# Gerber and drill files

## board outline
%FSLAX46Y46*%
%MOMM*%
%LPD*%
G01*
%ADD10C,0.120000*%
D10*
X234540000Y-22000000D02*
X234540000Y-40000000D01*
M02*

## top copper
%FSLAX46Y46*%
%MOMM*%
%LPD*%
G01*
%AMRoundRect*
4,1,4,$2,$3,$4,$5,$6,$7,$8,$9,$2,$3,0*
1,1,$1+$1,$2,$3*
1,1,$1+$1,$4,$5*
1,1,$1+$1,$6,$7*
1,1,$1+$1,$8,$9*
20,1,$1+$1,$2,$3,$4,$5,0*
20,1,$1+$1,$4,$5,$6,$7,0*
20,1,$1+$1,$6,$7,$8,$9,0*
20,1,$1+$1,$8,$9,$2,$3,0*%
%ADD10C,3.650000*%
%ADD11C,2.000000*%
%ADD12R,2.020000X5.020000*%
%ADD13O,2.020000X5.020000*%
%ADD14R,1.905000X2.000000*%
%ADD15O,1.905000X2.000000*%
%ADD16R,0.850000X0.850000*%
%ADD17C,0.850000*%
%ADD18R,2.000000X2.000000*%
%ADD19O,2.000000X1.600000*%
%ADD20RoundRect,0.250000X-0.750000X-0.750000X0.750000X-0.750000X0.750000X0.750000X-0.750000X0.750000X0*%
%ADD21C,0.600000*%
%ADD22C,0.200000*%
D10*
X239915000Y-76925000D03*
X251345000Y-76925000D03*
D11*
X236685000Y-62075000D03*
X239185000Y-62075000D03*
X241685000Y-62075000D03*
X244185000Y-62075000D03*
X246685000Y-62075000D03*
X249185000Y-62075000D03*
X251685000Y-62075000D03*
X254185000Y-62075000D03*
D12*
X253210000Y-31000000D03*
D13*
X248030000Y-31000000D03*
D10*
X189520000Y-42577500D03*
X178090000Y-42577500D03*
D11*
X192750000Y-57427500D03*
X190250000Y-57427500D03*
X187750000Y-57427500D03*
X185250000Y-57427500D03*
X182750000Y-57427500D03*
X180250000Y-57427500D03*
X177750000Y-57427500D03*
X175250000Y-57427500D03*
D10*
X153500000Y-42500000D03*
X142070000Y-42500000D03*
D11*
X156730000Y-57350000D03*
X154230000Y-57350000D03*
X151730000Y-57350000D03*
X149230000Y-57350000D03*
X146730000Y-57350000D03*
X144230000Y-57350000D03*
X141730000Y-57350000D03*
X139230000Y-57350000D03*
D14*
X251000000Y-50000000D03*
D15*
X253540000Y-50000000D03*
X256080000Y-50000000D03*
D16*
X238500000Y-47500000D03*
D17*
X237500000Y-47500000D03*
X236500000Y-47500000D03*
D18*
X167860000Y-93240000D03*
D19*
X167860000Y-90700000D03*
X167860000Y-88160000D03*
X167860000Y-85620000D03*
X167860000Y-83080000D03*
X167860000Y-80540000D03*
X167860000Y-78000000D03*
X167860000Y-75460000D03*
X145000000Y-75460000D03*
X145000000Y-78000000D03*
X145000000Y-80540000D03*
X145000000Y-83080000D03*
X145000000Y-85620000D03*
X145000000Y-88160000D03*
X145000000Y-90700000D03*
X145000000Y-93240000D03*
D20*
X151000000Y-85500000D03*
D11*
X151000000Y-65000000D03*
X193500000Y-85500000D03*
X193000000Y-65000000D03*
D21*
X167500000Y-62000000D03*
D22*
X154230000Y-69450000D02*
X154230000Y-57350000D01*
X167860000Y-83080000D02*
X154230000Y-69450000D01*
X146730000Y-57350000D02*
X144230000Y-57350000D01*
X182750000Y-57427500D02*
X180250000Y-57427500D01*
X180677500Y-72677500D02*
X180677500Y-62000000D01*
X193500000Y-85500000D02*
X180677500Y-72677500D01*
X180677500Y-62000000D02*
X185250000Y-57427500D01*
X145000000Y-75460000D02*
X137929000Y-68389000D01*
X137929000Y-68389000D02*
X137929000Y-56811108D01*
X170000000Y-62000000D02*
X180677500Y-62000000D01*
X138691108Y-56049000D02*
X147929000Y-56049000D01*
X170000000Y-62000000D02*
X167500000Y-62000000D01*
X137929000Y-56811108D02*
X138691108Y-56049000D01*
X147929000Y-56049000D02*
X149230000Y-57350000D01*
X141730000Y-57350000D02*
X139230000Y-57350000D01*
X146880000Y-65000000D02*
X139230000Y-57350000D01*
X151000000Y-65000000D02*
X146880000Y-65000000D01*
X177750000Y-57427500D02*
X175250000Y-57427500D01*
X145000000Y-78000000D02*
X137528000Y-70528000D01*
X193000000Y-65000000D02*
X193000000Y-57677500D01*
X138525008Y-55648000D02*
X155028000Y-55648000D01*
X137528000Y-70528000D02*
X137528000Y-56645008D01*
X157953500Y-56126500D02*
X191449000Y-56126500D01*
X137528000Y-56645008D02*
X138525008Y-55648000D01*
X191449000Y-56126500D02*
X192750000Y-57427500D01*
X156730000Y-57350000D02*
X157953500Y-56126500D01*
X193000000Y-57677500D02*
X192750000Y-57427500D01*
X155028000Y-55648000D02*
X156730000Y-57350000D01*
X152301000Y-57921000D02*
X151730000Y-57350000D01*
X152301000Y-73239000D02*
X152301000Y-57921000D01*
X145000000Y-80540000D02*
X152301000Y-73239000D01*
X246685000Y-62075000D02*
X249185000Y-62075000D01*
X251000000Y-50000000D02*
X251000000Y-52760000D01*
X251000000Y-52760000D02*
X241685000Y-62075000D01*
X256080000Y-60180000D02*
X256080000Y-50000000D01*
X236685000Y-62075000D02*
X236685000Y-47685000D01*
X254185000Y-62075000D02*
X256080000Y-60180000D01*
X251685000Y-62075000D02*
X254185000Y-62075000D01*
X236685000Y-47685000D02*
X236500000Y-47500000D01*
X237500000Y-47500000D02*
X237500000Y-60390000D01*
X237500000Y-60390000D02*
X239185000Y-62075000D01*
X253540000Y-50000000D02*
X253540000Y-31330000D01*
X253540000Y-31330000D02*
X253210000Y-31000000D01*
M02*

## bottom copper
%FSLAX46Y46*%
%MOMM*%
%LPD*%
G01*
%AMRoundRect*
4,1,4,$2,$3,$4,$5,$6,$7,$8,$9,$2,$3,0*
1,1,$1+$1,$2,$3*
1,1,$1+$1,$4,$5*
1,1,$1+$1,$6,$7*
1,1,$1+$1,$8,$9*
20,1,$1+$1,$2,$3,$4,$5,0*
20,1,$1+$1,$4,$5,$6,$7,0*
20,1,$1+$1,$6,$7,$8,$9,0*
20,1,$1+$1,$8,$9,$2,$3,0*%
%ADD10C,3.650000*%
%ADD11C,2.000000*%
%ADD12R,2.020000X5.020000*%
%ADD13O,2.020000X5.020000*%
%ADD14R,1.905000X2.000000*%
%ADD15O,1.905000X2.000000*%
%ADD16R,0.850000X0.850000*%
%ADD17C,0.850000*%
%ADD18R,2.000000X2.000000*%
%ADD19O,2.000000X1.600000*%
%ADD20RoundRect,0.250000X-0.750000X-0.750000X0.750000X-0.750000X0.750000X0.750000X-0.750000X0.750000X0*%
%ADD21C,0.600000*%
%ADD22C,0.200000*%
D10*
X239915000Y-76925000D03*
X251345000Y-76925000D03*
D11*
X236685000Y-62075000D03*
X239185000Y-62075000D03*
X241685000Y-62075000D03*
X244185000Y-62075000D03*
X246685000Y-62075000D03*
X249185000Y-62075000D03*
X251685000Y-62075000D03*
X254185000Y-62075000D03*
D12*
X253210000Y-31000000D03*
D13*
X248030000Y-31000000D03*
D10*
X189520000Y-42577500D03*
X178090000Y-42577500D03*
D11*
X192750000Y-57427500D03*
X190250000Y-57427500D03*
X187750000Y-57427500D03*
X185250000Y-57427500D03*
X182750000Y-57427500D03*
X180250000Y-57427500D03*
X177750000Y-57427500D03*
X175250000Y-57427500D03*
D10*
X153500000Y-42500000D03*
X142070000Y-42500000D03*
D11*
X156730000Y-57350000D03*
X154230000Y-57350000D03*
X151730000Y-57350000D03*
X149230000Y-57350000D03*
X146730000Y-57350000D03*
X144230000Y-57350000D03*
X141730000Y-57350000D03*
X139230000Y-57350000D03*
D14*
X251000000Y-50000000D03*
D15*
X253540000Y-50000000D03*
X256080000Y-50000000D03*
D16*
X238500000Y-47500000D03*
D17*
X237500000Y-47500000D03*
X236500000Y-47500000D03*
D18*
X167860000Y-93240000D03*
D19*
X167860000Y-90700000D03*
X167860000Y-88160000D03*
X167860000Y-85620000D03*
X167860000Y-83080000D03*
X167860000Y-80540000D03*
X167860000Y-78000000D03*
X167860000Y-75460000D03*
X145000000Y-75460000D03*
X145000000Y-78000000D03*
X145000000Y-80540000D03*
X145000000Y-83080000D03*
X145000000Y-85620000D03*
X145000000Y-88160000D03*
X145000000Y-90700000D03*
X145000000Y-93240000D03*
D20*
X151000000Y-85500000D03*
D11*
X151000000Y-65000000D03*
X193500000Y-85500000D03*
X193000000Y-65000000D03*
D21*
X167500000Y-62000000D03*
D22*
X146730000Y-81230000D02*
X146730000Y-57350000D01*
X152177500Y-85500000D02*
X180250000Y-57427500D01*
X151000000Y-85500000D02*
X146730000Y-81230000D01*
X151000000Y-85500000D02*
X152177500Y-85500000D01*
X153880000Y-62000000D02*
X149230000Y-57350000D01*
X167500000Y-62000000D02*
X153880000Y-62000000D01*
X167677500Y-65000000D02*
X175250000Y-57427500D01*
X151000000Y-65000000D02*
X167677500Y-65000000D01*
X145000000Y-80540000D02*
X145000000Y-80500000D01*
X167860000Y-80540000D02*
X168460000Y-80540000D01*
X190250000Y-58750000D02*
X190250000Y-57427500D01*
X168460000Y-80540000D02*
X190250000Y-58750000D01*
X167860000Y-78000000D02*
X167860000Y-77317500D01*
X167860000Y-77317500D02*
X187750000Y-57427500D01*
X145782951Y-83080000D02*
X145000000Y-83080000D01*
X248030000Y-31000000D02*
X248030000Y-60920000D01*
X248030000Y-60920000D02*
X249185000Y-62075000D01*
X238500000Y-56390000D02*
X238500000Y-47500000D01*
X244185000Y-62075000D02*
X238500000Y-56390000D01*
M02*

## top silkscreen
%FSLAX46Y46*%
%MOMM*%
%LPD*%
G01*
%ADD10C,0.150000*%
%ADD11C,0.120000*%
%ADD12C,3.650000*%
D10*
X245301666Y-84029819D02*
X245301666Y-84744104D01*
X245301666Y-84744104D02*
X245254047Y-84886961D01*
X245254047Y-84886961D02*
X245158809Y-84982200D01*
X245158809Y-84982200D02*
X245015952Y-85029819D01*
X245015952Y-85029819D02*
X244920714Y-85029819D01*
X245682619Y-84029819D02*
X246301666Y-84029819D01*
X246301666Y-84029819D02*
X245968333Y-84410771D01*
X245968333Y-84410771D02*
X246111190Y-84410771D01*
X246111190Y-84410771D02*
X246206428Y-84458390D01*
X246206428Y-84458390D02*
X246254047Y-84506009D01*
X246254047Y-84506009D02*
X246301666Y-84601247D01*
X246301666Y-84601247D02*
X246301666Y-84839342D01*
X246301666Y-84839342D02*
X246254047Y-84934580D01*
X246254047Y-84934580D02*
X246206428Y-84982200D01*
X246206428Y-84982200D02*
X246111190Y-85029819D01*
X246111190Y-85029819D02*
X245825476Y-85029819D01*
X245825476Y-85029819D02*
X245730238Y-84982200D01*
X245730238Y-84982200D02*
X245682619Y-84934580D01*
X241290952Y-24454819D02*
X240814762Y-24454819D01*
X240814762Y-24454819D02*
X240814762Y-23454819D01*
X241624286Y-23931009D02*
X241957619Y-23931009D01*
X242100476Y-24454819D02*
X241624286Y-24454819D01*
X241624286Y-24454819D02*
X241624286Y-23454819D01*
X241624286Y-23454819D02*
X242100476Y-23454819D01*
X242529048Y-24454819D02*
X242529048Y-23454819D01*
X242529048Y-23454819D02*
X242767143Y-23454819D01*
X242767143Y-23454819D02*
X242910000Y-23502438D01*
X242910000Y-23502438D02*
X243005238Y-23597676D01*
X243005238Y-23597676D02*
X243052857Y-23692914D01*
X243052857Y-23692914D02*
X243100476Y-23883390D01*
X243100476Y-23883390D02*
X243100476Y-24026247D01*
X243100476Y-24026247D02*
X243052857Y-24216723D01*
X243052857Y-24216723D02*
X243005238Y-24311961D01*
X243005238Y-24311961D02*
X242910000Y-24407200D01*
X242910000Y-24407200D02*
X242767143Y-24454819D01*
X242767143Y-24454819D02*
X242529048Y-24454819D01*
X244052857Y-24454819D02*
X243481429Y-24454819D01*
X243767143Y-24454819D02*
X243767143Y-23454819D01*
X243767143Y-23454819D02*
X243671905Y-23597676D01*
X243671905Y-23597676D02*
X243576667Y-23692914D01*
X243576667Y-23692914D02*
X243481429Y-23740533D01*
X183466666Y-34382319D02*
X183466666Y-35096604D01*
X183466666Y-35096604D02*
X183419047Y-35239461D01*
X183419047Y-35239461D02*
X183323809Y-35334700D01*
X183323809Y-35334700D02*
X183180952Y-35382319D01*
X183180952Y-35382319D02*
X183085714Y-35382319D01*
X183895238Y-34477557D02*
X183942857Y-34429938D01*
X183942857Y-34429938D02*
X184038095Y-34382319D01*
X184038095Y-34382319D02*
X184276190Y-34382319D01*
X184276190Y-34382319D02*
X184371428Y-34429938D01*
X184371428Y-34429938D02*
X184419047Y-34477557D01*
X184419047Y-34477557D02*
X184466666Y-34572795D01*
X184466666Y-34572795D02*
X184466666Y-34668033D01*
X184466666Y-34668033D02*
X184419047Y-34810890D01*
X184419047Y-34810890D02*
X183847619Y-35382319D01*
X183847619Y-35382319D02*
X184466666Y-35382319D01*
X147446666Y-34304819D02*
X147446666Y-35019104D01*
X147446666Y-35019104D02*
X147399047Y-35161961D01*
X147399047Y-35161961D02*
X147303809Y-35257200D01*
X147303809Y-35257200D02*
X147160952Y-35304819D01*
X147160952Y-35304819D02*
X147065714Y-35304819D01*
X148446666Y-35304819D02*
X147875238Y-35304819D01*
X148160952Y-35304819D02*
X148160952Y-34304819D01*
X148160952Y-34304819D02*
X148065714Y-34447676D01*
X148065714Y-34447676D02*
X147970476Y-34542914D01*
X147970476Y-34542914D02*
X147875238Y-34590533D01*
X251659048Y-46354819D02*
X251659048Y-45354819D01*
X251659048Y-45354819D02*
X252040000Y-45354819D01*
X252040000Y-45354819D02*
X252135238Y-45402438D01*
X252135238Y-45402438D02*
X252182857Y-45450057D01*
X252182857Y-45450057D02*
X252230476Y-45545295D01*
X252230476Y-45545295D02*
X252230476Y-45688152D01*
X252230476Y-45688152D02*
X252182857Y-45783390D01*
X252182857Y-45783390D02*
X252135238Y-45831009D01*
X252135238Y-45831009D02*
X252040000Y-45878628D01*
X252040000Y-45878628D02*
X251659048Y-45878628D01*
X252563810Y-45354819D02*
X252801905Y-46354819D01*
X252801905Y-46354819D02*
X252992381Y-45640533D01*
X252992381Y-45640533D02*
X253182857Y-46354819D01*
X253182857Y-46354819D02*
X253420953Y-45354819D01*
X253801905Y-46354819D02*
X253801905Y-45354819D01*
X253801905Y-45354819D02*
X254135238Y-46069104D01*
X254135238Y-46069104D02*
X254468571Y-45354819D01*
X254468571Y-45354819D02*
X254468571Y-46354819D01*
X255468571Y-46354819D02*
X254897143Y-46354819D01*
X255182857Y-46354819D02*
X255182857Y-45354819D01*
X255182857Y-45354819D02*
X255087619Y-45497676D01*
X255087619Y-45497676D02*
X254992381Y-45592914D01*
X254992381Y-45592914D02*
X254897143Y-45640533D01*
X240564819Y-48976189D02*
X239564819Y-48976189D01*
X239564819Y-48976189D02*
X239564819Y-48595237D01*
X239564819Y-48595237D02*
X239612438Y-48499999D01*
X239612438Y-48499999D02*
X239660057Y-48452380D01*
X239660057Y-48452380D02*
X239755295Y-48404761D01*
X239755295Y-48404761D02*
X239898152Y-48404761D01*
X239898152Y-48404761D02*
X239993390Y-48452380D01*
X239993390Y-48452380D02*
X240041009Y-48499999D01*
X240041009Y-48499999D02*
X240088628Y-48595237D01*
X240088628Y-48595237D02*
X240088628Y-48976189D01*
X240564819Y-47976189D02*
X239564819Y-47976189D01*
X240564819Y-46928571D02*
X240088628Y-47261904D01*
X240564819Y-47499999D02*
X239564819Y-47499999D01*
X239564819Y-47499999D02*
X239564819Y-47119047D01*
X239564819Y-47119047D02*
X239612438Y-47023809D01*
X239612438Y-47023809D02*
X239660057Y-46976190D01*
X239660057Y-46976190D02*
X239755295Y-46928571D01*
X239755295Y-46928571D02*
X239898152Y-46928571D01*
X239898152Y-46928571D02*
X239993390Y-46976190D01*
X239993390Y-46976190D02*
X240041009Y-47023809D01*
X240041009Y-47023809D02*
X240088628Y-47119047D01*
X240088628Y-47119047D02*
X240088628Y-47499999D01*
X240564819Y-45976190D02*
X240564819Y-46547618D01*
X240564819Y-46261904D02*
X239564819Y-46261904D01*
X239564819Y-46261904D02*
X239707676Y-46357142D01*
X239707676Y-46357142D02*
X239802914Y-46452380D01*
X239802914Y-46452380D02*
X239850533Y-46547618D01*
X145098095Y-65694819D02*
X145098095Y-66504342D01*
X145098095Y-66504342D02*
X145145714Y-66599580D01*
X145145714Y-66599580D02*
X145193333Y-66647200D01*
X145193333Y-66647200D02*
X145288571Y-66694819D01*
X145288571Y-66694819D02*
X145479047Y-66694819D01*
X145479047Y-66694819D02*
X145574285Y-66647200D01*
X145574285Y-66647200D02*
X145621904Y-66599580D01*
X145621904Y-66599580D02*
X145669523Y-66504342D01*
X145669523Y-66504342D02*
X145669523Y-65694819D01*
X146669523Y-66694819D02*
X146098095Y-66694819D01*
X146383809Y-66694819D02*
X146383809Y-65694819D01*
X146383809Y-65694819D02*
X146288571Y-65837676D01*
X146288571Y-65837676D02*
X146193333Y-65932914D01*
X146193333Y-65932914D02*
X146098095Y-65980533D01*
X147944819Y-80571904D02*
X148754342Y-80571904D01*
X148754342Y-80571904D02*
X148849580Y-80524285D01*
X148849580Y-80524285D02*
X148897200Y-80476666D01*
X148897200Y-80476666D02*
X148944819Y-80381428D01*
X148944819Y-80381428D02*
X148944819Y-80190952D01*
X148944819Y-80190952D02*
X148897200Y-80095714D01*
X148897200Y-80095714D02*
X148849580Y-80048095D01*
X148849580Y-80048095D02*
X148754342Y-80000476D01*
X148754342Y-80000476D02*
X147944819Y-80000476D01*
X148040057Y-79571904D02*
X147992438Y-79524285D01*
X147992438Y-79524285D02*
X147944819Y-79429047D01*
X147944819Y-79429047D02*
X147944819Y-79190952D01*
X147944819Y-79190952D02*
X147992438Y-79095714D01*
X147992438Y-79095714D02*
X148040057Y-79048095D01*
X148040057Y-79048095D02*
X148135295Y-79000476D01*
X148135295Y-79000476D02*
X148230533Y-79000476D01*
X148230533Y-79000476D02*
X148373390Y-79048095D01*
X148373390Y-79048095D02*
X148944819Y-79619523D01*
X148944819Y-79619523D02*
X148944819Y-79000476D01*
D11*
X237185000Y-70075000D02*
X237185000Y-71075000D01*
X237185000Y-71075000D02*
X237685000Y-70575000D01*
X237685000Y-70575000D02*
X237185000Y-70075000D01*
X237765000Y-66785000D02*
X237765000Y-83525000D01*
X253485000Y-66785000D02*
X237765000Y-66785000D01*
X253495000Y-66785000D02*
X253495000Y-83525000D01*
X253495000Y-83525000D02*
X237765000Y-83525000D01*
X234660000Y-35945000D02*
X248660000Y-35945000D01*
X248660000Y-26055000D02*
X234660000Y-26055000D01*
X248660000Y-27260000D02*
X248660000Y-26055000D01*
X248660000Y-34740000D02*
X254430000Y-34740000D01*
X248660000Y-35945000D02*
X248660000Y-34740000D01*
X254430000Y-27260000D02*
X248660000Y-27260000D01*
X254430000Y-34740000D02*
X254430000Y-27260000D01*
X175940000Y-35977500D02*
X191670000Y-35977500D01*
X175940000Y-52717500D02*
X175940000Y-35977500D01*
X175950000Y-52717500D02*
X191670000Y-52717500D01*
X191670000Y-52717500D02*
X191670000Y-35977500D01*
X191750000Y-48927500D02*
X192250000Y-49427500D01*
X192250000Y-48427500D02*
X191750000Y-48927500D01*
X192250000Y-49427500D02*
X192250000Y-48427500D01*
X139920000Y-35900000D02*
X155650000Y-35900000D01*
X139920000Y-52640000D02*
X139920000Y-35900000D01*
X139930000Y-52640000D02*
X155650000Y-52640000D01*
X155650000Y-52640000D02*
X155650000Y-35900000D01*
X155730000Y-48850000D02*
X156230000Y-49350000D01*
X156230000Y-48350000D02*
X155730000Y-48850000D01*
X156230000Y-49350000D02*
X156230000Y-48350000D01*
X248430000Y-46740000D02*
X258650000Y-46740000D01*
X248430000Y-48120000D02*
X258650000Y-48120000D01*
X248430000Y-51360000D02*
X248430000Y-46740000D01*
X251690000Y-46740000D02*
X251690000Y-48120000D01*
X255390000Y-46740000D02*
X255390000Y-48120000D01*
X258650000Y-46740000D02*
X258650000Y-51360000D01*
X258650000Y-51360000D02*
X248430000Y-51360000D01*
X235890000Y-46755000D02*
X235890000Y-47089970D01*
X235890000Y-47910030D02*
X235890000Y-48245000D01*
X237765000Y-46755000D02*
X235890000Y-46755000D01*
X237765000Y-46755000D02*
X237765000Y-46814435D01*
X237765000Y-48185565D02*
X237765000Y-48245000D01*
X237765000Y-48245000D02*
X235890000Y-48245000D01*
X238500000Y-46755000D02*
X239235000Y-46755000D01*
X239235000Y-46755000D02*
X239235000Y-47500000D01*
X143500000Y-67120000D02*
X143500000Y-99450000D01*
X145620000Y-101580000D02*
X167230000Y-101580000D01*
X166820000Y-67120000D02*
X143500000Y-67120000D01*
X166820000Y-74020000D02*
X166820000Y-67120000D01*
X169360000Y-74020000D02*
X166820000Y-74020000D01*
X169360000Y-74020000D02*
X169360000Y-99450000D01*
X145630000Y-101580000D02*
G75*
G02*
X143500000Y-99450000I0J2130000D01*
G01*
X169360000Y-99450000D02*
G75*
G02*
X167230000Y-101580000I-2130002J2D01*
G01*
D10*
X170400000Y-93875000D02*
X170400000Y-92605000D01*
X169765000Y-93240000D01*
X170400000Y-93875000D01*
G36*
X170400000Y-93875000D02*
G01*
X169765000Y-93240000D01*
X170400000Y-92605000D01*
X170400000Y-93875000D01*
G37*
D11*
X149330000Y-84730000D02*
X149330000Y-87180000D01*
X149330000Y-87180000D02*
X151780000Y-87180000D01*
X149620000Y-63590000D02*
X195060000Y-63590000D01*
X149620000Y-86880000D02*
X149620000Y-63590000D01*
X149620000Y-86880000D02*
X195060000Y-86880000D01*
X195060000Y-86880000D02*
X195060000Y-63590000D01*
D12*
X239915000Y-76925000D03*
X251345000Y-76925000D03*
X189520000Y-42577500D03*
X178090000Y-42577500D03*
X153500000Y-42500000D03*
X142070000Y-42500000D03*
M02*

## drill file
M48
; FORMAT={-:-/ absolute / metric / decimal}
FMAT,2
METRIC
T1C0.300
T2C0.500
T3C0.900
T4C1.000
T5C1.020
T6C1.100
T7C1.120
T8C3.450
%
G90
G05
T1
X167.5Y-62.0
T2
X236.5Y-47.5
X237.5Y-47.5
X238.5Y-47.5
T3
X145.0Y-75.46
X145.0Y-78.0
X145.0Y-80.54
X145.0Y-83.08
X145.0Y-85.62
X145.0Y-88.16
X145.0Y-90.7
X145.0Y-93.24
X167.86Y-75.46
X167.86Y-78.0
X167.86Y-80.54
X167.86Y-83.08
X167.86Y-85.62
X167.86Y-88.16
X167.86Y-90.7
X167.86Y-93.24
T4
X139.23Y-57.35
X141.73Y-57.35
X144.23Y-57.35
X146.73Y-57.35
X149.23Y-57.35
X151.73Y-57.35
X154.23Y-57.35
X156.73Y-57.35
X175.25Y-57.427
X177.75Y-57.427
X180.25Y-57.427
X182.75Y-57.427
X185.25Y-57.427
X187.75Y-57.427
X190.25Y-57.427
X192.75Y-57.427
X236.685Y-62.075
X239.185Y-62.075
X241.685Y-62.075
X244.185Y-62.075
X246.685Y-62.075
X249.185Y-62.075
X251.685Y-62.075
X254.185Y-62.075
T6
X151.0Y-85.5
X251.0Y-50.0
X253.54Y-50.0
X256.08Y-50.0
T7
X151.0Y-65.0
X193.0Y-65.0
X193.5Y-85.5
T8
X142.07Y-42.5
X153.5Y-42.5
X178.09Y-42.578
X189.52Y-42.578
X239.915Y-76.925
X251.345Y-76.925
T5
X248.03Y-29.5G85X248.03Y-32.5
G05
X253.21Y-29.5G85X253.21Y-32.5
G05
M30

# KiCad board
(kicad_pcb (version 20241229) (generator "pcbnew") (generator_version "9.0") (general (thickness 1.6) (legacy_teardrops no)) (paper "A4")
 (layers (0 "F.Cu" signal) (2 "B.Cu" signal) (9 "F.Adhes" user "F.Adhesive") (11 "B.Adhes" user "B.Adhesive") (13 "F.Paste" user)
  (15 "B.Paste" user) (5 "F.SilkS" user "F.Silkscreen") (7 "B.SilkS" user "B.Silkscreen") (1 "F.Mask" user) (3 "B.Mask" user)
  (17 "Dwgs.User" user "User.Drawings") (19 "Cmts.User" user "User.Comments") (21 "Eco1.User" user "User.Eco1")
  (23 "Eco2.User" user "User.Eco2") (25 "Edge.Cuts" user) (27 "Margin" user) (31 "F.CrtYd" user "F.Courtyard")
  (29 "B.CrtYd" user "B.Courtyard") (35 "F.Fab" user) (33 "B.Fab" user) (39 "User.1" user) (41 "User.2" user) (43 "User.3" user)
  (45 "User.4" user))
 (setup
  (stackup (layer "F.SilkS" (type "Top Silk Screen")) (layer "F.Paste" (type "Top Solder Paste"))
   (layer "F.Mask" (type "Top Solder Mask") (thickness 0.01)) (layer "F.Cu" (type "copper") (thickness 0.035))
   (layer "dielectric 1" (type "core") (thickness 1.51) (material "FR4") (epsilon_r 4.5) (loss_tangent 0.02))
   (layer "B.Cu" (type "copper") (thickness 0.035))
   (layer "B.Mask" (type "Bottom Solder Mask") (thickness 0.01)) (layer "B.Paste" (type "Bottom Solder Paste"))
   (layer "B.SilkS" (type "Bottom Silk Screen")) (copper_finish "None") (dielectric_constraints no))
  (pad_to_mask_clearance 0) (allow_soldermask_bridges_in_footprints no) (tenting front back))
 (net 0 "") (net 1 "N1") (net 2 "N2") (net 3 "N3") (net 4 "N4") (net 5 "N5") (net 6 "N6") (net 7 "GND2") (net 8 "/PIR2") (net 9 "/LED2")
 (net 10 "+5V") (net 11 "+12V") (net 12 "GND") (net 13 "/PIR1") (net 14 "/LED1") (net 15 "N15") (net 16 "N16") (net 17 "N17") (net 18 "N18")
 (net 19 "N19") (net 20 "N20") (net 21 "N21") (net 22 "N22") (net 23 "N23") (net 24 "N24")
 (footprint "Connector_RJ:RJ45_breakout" (layer "F.Cu") (at 241.185 70.575)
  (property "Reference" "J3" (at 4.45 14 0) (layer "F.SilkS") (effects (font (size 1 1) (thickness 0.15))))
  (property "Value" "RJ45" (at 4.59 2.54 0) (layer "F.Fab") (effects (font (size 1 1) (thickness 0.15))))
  (fp_line (start -4 -0.5) (end -4 0.5) (stroke (width 0.12) (type solid)) (layer "F.SilkS"))
  (fp_line (start -4 0.5) (end -3.5 0) (stroke (width 0.12) (type solid)) (layer "F.SilkS"))
  (fp_line (start -3.5 0) (end -4 -0.5) (stroke (width 0.12) (type solid)) (layer "F.SilkS"))
  (fp_line (start -3.42 -3.79) (end -3.42 12.95) (stroke (width 0.12) (type solid)) (layer "F.SilkS"))
  (fp_line (start 12.3 -3.79) (end -3.42 -3.79) (stroke (width 0.12) (type solid)) (layer "F.SilkS"))
  (fp_line (start 12.31 -3.79) (end 12.31 12.95) (stroke (width 0.12) (type solid)) (layer "F.SilkS"))
  (fp_line (start 12.31 12.95) (end -3.42 12.95) (stroke (width 0.12) (type solid)) (layer "F.SilkS"))
  (pad "" np_thru_hole circle (at -1.27 6.35) (size 3.65 3.65) (drill 3.45) (layers "*.Cu" "*.SilkS" "*.Mask"))
  (pad "" np_thru_hole circle (at 10.16 6.35) (size 3.65 3.65) (drill 3.45) (layers "*.Cu" "*.SilkS" "*.Mask"))
  (pad "1" thru_hole circle (at -4.5 -8.5) (size 2 2) (drill 1) (layers "*.Cu" "*.Mask") (remove_unused_layers no) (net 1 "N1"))
  (pad "2" thru_hole circle (at -2 -8.5) (size 2 2) (drill 1) (layers "*.Cu" "*.Mask") (remove_unused_layers no) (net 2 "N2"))
  (pad "3" thru_hole circle (at 0.5 -8.5) (size 2 2) (drill 1) (layers "*.Cu" "*.Mask") (remove_unused_layers no) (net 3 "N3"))
  (pad "4" thru_hole circle (at 3 -8.5) (size 2 2) (drill 1) (layers "*.Cu" "*.Mask") (remove_unused_layers no) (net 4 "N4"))
  (pad "5" thru_hole circle (at 5.5 -8.5) (size 2 2) (drill 1) (layers "*.Cu" "*.Mask") (remove_unused_layers no) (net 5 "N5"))
  (pad "6" thru_hole circle (at 8 -8.5) (size 2 2) (drill 1) (layers "*.Cu" "*.Mask") (remove_unused_layers no) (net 5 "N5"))
  (pad "7" thru_hole circle (at 10.5 -8.5) (size 2 2) (drill 1) (layers "*.Cu" "*.Mask") (remove_unused_layers no) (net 1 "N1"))
  (pad "8" thru_hole circle (at 13 -8.5) (size 2 2) (drill 1) (layers "*.Cu" "*.Mask") (remove_unused_layers no) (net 1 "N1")))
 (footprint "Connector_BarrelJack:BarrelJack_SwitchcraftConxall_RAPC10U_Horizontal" (layer "F.Cu") (at 253.21 31)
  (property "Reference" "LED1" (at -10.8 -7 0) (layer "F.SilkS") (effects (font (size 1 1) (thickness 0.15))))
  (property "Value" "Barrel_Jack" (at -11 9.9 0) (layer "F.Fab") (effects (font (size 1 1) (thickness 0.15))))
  (fp_line (start -18.55 4.945) (end -4.55 4.945) (stroke (width 0.12) (type solid)) (layer "F.SilkS"))
  (fp_line (start -4.55 -4.945) (end -18.55 -4.945) (stroke (width 0.12) (type solid)) (layer "F.SilkS"))
  (fp_line (start -4.55 -3.74) (end -4.55 -4.945) (stroke (width 0.12) (type solid)) (layer "F.SilkS"))
  (fp_line (start -4.55 3.74) (end 1.22 3.74) (stroke (width 0.12) (type solid)) (layer "F.SilkS"))
  (fp_line (start -4.55 4.945) (end -4.55 3.74) (stroke (width 0.12) (type solid)) (layer "F.SilkS"))
  (fp_line (start 1.22 -3.74) (end -4.55 -3.74) (stroke (width 0.12) (type solid)) (layer "F.SilkS"))
  (fp_line (start 1.22 3.74) (end 1.22 -3.74) (stroke (width 0.12) (type solid)) (layer "F.SilkS"))
  (fp_line (start -18.67 -9) (end -18.67 9) (stroke (width 0.12) (type solid)) (layer "Edge.Cuts"))
  (pad "1" thru_hole rect (at 0 0) (size 2.02 5.02) (drill oval 1.02 4.02) (layers "*.Cu" "*.Mask") (remove_unused_layers no) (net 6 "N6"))
  (pad "2" thru_hole oval (at -5.18 0) (size 2.02 5.02) (drill oval 1.02 4.02) (layers "*.Cu" "*.Mask") (remove_unused_layers no)
   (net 5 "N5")))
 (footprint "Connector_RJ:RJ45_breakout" (layer "F.Cu") (at 188.25 48.9275 180)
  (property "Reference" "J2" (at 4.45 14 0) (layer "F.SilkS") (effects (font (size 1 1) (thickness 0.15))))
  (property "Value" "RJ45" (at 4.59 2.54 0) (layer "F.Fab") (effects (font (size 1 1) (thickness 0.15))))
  (fp_line (start 12.31 12.95) (end -3.42 12.95) (stroke (width 0.12) (type solid)) (layer "F.SilkS"))
  (fp_line (start 12.31 -3.79) (end 12.31 12.95) (stroke (width 0.12) (type solid)) (layer "F.SilkS"))
  (fp_line (start 12.3 -3.79) (end -3.42 -3.79) (stroke (width 0.12) (type solid)) (layer "F.SilkS"))
  (fp_line (start -3.42 -3.79) (end -3.42 12.95) (stroke (width 0.12) (type solid)) (layer "F.SilkS"))
  (fp_line (start -3.5 0) (end -4 -0.5) (stroke (width 0.12) (type solid)) (layer "F.SilkS"))
  (fp_line (start -4 0.5) (end -3.5 0) (stroke (width 0.12) (type solid)) (layer "F.SilkS"))
  (fp_line (start -4 -0.5) (end -4 0.5) (stroke (width 0.12) (type solid)) (layer "F.SilkS"))
  (pad "" np_thru_hole circle (at -1.27 6.35 180) (size 3.65 3.65) (drill 3.45) (layers "*.Cu" "*.SilkS" "*.Mask"))
  (pad "" np_thru_hole circle (at 10.16 6.35 180) (size 3.65 3.65) (drill 3.45) (layers "*.Cu" "*.SilkS" "*.Mask"))
  (pad "1" thru_hole circle (at -4.5 -8.5 180) (size 2 2) (drill 1) (layers "*.Cu" "*.Mask") (remove_unused_layers no) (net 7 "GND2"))
  (pad "2" thru_hole circle (at -2 -8.5 180) (size 2 2) (drill 1) (layers "*.Cu" "*.Mask") (remove_unused_layers no) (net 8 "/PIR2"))
  (pad "3" thru_hole circle (at 0.5 -8.5 180) (size 2 2) (drill 1) (layers "*.Cu" "*.Mask") (remove_unused_layers no) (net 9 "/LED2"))
  (pad "4" thru_hole circle (at 3 -8.5 180) (size 2 2) (drill 1) (layers "*.Cu" "*.Mask") (remove_unused_layers no) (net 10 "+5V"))
  (pad "5" thru_hole circle (at 5.5 -8.5 180) (size 2 2) (drill 1) (layers "*.Cu" "*.Mask") (remove_unused_layers no) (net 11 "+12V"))
  (pad "6" thru_hole circle (at 8 -8.5 180) (size 2 2) (drill 1) (layers "*.Cu" "*.Mask") (remove_unused_layers no) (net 11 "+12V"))
  (pad "7" thru_hole circle (at 10.5 -8.5 180) (size 2 2) (drill 1) (layers "*.Cu" "*.Mask") (remove_unused_layers no) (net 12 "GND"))
  (pad "8" thru_hole circle (at 13 -8.5 180) (size 2 2) (drill 1) (layers "*.Cu" "*.Mask") (remove_unused_layers no) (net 12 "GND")))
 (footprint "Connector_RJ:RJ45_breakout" (layer "F.Cu") (at 152.23 48.85 180)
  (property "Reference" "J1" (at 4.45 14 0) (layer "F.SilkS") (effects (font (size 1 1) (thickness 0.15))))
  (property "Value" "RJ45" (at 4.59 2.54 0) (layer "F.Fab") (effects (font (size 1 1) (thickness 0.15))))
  (fp_line (start 12.31 12.95) (end -3.42 12.95) (stroke (width 0.12) (type solid)) (layer "F.SilkS"))
  (fp_line (start 12.31 -3.79) (end 12.31 12.95) (stroke (width 0.12) (type solid)) (layer "F.SilkS"))
  (fp_line (start 12.3 -3.79) (end -3.42 -3.79) (stroke (width 0.12) (type solid)) (layer "F.SilkS"))
  (fp_line (start -3.42 -3.79) (end -3.42 12.95) (stroke (width 0.12) (type solid)) (layer "F.SilkS"))
  (fp_line (start -3.5 0) (end -4 -0.5) (stroke (width 0.12) (type solid)) (layer "F.SilkS"))
  (fp_line (start -4 0.5) (end -3.5 0) (stroke (width 0.12) (type solid)) (layer "F.SilkS"))
  (fp_line (start -4 -0.5) (end -4 0.5) (stroke (width 0.12) (type solid)) (layer "F.SilkS"))
  (pad "" np_thru_hole circle (at -1.27 6.35 180) (size 3.65 3.65) (drill 3.45) (layers "*.Cu" "*.SilkS" "*.Mask"))
  (pad "" np_thru_hole circle (at 10.16 6.35 180) (size 3.65 3.65) (drill 3.45) (layers "*.Cu" "*.SilkS" "*.Mask"))
  (pad "1" thru_hole circle (at -4.5 -8.5 180) (size 2 2) (drill 1) (layers "*.Cu" "*.Mask") (remove_unused_layers no) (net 7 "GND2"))
  (pad "2" thru_hole circle (at -2 -8.5 180) (size 2 2) (drill 1) (layers "*.Cu" "*.Mask") (remove_unused_layers no) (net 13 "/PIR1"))
  (pad "3" thru_hole circle (at 0.5 -8.5 180) (size 2 2) (drill 1) (layers "*.Cu" "*.Mask") (remove_unused_layers no) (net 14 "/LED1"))
  (pad "4" thru_hole circle (at 3 -8.5 180) (size 2 2) (drill 1) (layers "*.Cu" "*.Mask") (remove_unused_layers no) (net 10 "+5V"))
  (pad "5" thru_hole circle (at 5.5 -8.5 180) (size 2 2) (drill 1) (layers "*.Cu" "*.Mask") (remove_unused_layers no) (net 11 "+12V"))
  (pad "6" thru_hole circle (at 8 -8.5 180) (size 2 2) (drill 1) (layers "*.Cu" "*.Mask") (remove_unused_layers no) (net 11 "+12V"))
  (pad "7" thru_hole circle (at 10.5 -8.5 180) (size 2 2) (drill 1) (layers "*.Cu" "*.Mask") (remove_unused_layers no) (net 12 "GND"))
  (pad "8" thru_hole circle (at 13 -8.5 180) (size 2 2) (drill 1) (layers "*.Cu" "*.Mask") (remove_unused_layers no) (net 12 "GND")))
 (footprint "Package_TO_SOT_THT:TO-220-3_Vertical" (layer "F.Cu") (at 251 50)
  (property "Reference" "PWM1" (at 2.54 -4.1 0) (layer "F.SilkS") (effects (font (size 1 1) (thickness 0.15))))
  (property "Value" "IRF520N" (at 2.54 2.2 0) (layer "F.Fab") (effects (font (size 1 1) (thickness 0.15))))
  (fp_line (start -2.57 -3.26) (end 7.65 -3.26) (stroke (width 0.12) (type solid)) (layer "F.SilkS"))
  (fp_line (start -2.57 -1.88) (end 7.65 -1.88) (stroke (width 0.12) (type solid)) (layer "F.SilkS"))
  (fp_line (start -2.57 1.36) (end -2.57 -3.26) (stroke (width 0.12) (type solid)) (layer "F.SilkS"))
  (fp_line (start 0.69 -3.26) (end 0.69 -1.88) (stroke (width 0.12) (type solid)) (layer "F.SilkS"))
  (fp_line (start 4.39 -3.26) (end 4.39 -1.88) (stroke (width 0.12) (type solid)) (layer "F.SilkS"))
  (fp_line (start 7.65 -3.26) (end 7.65 1.36) (stroke (width 0.12) (type solid)) (layer "F.SilkS"))
  (fp_line (start 7.65 1.36) (end -2.57 1.36) (stroke (width 0.12) (type solid)) (layer "F.SilkS"))
  (pad "1" thru_hole rect (at 0 0) (size 1.905 2) (drill 1.1) (layers "*.Cu" "*.Mask") (remove_unused_layers no) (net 3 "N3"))
  (pad "2" thru_hole oval (at 2.54 0) (size 1.905 2) (drill 1.1) (layers "*.Cu" "*.Mask") (remove_unused_layers no) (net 6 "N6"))
  (pad "3" thru_hole oval (at 5.08 0) (size 1.905 2) (drill 1.1) (layers "*.Cu" "*.Mask") (remove_unused_layers no) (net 1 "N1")))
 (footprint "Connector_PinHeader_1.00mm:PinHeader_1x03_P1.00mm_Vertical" (layer "F.Cu") (at 238.5 47.5 -90)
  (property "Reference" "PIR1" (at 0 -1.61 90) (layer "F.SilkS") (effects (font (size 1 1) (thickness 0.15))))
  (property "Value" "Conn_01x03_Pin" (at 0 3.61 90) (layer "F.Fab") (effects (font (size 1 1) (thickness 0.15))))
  (fp_line (start -0.745 2.61) (end -0.41003 2.61) (stroke (width 0.12) (type solid)) (layer "F.SilkS"))
  (fp_line (start 0.41003 2.61) (end 0.745 2.61) (stroke (width 0.12) (type solid)) (layer "F.SilkS"))
  (fp_line (start -0.745 0.735) (end -0.745 2.61) (stroke (width 0.12) (type solid)) (layer "F.SilkS"))
  (fp_line (start -0.745 0.735) (end -0.685565 0.735) (stroke (width 0.12) (type solid)) (layer "F.SilkS"))
  (fp_line (start 0.685565 0.735) (end 0.745 0.735) (stroke (width 0.12) (type solid)) (layer "F.SilkS"))
  (fp_line (start 0.745 0.735) (end 0.745 2.61) (stroke (width 0.12) (type solid)) (layer "F.SilkS"))
  (fp_line (start -0.745 0) (end -0.745 -0.735) (stroke (width 0.12) (type solid)) (layer "F.SilkS"))
  (fp_line (start -0.745 -0.735) (end 0 -0.735) (stroke (width 0.12) (type solid)) (layer "F.SilkS"))
  (pad "1" thru_hole rect (at 0 0 270) (size 0.85 0.85) (drill 0.5) (layers "*.Cu" "*.Mask") (remove_unused_layers no) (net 4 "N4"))
  (pad "2" thru_hole circle (at 0 1 270) (size 0.85 0.85) (drill 0.5) (layers "*.Cu" "*.Mask") (remove_unused_layers no) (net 2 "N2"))
  (pad "3" thru_hole circle (at 0 2 270) (size 0.85 0.85) (drill 0.5) (layers "*.Cu" "*.Mask") (remove_unused_layers no) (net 1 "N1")))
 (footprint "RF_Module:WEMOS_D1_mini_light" (layer "F.Cu") (at 167.86 93.24 180)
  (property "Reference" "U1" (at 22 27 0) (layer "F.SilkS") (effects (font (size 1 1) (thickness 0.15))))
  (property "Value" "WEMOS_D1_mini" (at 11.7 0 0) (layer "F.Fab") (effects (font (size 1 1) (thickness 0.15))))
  (fp_line (start 24.36 26.12) (end 24.36 -6.21) (stroke (width 0.12) (type solid)) (layer "F.SilkS"))
  (fp_line (start 22.24 -8.34) (end 0.63 -8.34) (stroke (width 0.12) (type solid)) (layer "F.SilkS"))
  (fp_line (start 1.04 26.12) (end 24.36 26.12) (stroke (width 0.12) (type solid)) (layer "F.SilkS"))
  (fp_line (start 1.04 19.22) (end 1.04 26.12) (stroke (width 0.12) (type solid)) (layer "F.SilkS"))
  (fp_line (start -1.5 19.22) (end 1.04 19.22) (stroke (width 0.12) (type solid)) (layer "F.SilkS"))
  (fp_line (start -1.5 19.22) (end -1.5 -6.21) (stroke (width 0.12) (type solid)) (layer "F.SilkS"))
  (fp_arc (start 22.23 -8.34) (mid 23.736137 -7.716137) (end 24.36 -6.21) (stroke (width 0.12) (type solid)) (layer "F.SilkS"))
  (fp_arc (start -1.5 -6.21) (mid -0.876137 -7.716137) (end 0.63 -8.34) (stroke (width 0.12) (type solid)) (layer "F.SilkS"))
  (fp_poly (pts (xy -2.54 -0.635) (xy -2.54 0.635) (xy -1.905 0)) (stroke (width 0.15) (type solid)) (fill yes) (layer "F.SilkS"))
  (pad "1" thru_hole rect (at 0 0 180) (size 2 2) (drill 0.9) (layers "*.Cu" "*.Mask") (remove_unused_layers no) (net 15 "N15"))
  (pad "2" thru_hole oval (at 0 2.54 180) (size 2 1.6) (drill 0.9) (layers "*.Cu" "*.Mask") (remove_unused_layers no) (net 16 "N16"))
  (pad "3" thru_hole oval (at 0 5.08 180) (size 2 1.6) (drill 0.9) (layers "*.Cu" "*.Mask") (remove_unused_layers no) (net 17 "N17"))
  (pad "4" thru_hole oval (at 0 7.62 180) (size 2 1.6) (drill 0.9) (layers "*.Cu" "*.Mask") (remove_unused_layers no) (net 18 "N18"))
  (pad "5" thru_hole oval (at 0 10.16 180) (size 2 1.6) (drill 0.9) (layers "*.Cu" "*.Mask") (remove_unused_layers no) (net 13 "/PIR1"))
  (pad "6" thru_hole oval (at 0 12.7 180) (size 2 1.6) (drill 0.9) (layers "*.Cu" "*.Mask") (remove_unused_layers no) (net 8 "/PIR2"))
  (pad "7" thru_hole oval (at 0 15.24 180) (size 2 1.6) (drill 0.9) (layers "*.Cu" "*.Mask") (remove_unused_layers no) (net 9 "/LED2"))
  (pad "8" thru_hole oval (at 0 17.78 180) (size 2 1.6) (drill 0.9) (layers "*.Cu" "*.Mask") (remove_unused_layers no) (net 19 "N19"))
  (pad "9" thru_hole oval (at 22.86 17.78 180) (size 2 1.6) (drill 0.9) (layers "*.Cu" "*.Mask") (remove_unused_layers no) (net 10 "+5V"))
  (pad "10" thru_hole oval (at 22.86 15.24 180) (size 2 1.6) (drill 0.9) (layers "*.Cu" "*.Mask") (remove_unused_layers no) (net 7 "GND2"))
  (pad "11" thru_hole oval (at 22.86 12.7 180) (size 2 1.6) (drill 0.9) (layers "*.Cu" "*.Mask") (remove_unused_layers no) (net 14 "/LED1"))
  (pad "12" thru_hole oval (at 22.86 10.16 180) (size 2 1.6) (drill 0.9) (layers "*.Cu" "*.Mask") (remove_unused_layers no) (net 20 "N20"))
  (pad "13" thru_hole oval (at 22.86 7.62 180) (size 2 1.6) (drill 0.9) (layers "*.Cu" "*.Mask") (remove_unused_layers no) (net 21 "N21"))
  (pad "14" thru_hole oval (at 22.86 5.08 180) (size 2 1.6) (drill 0.9) (layers "*.Cu" "*.Mask") (remove_unused_layers no) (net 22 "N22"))
  (pad "15" thru_hole oval (at 22.86 2.54 180) (size 2 1.6) (drill 0.9) (layers "*.Cu" "*.Mask") (remove_unused_layers no) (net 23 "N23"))
  (pad "16" thru_hole oval (at 22.86 0 180) (size 2 1.6) (drill 0.9) (layers "*.Cu" "*.Mask") (remove_unused_layers no) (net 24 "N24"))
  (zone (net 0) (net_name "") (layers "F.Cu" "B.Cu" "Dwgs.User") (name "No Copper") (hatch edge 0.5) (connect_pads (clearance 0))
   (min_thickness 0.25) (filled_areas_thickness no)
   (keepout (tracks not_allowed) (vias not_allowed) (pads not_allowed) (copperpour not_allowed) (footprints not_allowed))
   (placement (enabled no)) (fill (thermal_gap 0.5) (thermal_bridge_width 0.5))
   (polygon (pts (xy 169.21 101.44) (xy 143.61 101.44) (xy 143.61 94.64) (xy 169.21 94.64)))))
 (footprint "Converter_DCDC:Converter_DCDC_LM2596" (layer "F.Cu") (at 151 85.5 90)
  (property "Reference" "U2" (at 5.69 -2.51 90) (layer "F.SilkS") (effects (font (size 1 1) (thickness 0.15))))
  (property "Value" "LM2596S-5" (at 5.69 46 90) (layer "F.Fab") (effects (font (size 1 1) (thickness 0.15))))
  (fp_line (start 0.77 -1.67) (end -1.68 -1.67) (stroke (width 0.12) (type default)) (layer "F.SilkS"))
  (fp_line (start -1.68 -1.67) (end -1.68 0.78) (stroke (width 0.12) (type default)) (layer "F.SilkS"))
  (fp_line (start 21.91 -1.38) (end 21.91 44.06) (stroke (width 0.12) (type solid)) (layer "F.SilkS"))
  (fp_line (start -1.38 -1.38) (end 21.91 -1.38) (stroke (width 0.12) (type solid)) (layer "F.SilkS"))
  (fp_line (start -1.38 -1.38) (end -1.38 44.06) (stroke (width 0.12) (type solid)) (layer "F.SilkS"))
  (fp_line (start -1.38 44.06) (end 21.91 44.06) (stroke (width 0.12) (type solid)) (layer "F.SilkS"))
  (pad "1" thru_hole roundrect (at 0 0) (size 2 2) (drill 1.1) (layers "*.Cu" "*.Mask") (remove_unused_layers no) (roundrect_rratio 0.125)
   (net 11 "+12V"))
  (pad "2" thru_hole circle (at 20.5 0) (size 2 2) (drill 1.12) (layers "*.Cu" "*.Mask") (remove_unused_layers no) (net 12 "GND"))
  (pad "3" thru_hole circle (at 0 42.5) (size 2 2) (drill 1.12) (layers "*.Cu" "*.Mask") (remove_unused_layers no) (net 10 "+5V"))
  (pad "4" thru_hole circle (at 20.5 42) (size 2 2) (drill 1.12) (layers "*.Cu" "*.Mask") (remove_unused_layers no) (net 7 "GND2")))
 (segment (start 154.23 69.45) (end 154.23 57.35) (width 0.2) (layer "F.Cu") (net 13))
 (segment (start 167.86 83.08) (end 154.23 69.45) (width 0.2) (layer "F.Cu") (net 13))
 (segment (start 146.73 57.35) (end 144.23 57.35) (width 0.2) (layer "F.Cu") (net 11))
 (segment (start 182.75 57.4275) (end 180.25 57.4275) (width 0.2) (layer "F.Cu") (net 11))
 (segment (start 146.73 81.23) (end 146.73 57.35) (width 0.2) (layer "B.Cu") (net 11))
 (segment (start 152.1775 85.5) (end 180.25 57.4275) (width 0.2) (layer "B.Cu") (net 11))
 (segment (start 151 85.5) (end 146.73 81.23) (width 0.2) (layer "B.Cu") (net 11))
 (segment (start 151 85.5) (end 152.1775 85.5) (width 0.2) (layer "B.Cu") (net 11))
 (segment (start 180.6775 72.6775) (end 180.6775 62) (width 0.2) (layer "F.Cu") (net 10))
 (segment (start 193.5 85.5) (end 180.6775 72.6775) (width 0.2) (layer "F.Cu") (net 10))
 (segment (start 180.6775 62) (end 185.25 57.4275) (width 0.2) (layer "F.Cu") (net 10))
 (segment (start 145 75.46) (end 137.929 68.389) (width 0.2) (layer "F.Cu") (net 10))
 (segment (start 137.929 68.389) (end 137.929 56.811108) (width 0.2) (layer "F.Cu") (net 10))
 (segment (start 170 62) (end 180.6775 62) (width 0.2) (layer "F.Cu") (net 10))
 (segment (start 138.691108 56.049) (end 147.929 56.049) (width 0.2) (layer "F.Cu") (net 10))
 (segment (start 170 62) (end 167.5 62) (width 0.2) (layer "F.Cu") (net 10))
 (segment (start 137.929 56.811108) (end 138.691108 56.049) (width 0.2) (layer "F.Cu") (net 10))
 (segment (start 147.929 56.049) (end 149.23 57.35) (width 0.2) (layer "F.Cu") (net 10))
 (via (at 167.5 62) (size 0.6) (drill 0.3) (layers "F.Cu" "B.Cu") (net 10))
 (segment (start 153.88 62) (end 149.23 57.35) (width 0.2) (layer "B.Cu") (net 10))
 (segment (start 167.5 62) (end 153.88 62) (width 0.2) (layer "B.Cu") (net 10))
 (segment (start 141.73 57.35) (end 139.23 57.35) (width 0.2) (layer "F.Cu") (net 12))
 (segment (start 146.88 65) (end 139.23 57.35) (width 0.2) (layer "F.Cu") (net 12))
 (segment (start 151 65) (end 146.88 65) (width 0.2) (layer "F.Cu") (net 12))
 (segment (start 177.75 57.4275) (end 175.25 57.4275) (width 0.2) (layer "F.Cu") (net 12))
 (segment (start 167.6775 65) (end 175.25 57.4275) (width 0.2) (layer "B.Cu") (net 12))
 (segment (start 151 65) (end 167.6775 65) (width 0.2) (layer "B.Cu") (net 12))
 (segment (start 145 78) (end 137.528 70.528) (width 0.2) (layer "F.Cu") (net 7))
 (segment (start 193 65) (end 193 57.6775) (width 0.2) (layer "F.Cu") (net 7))
 (segment (start 138.525008 55.648) (end 155.028 55.648) (width 0.2) (layer "F.Cu") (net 7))
 (segment (start 137.528 70.528) (end 137.528 56.645008) (width 0.2) (layer "F.Cu") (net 7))
 (segment (start 157.9535 56.1265) (end 191.449 56.1265) (width 0.2) (layer "F.Cu") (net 7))
 (segment (start 137.528 56.645008) (end 138.525008 55.648) (width 0.2) (layer "F.Cu") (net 7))
 (segment (start 191.449 56.1265) (end 192.75 57.4275) (width 0.2) (layer "F.Cu") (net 7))
 (segment (start 156.73 57.35) (end 157.9535 56.1265) (width 0.2) (layer "F.Cu") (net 7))
 (segment (start 193 57.6775) (end 192.75 57.4275) (width 0.2) (layer "F.Cu") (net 7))
 (segment (start 155.028 55.648) (end 156.73 57.35) (width 0.2) (layer "F.Cu") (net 7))
 (segment (start 152.301 57.921) (end 151.73 57.35) (width 0.2) (layer "F.Cu") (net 14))
 (segment (start 152.301 73.239) (end 152.301 57.921) (width 0.2) (layer "F.Cu") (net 14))
 (segment (start 145 80.54) (end 152.301 73.239) (width 0.2) (layer "F.Cu") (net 14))
 (segment (start 145 80.54) (end 145 80.5) (width 0.2) (layer "B.Cu") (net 14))
 (segment (start 167.86 80.54) (end 168.46 80.54) (width 0.2) (layer "B.Cu") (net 8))
 (segment (start 190.25 58.75) (end 190.25 57.4275) (width 0.2) (layer "B.Cu") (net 8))
 (segment (start 168.46 80.54) (end 190.25 58.75) (width 0.2) (layer "B.Cu") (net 8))
 (segment (start 167.86 78) (end 167.86 77.3175) (width 0.2) (layer "B.Cu") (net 9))
 (segment (start 167.86 77.3175) (end 187.75 57.4275) (width 0.2) (layer "B.Cu") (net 9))
 (segment (start 145.782951 83.08) (end 145 83.08) (width 0.2) (layer "B.Cu") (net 20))
 (segment (start 246.685 62.075) (end 249.185 62.075) (width 0.2) (layer "F.Cu") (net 5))
 (segment (start 248.03 31) (end 248.03 60.92) (width 0.2) (layer "B.Cu") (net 5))
 (segment (start 248.03 60.92) (end 249.185 62.075) (width 0.2) (layer "B.Cu") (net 5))
 (segment (start 251 50) (end 251 52.76) (width 0.2) (layer "F.Cu") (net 3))
 (segment (start 251 52.76) (end 241.685 62.075) (width 0.2) (layer "F.Cu") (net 3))
 (segment (start 256.08 60.18) (end 256.08 50) (width 0.2) (layer "F.Cu") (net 1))
 (segment (start 236.685 62.075) (end 236.685 47.685) (width 0.2) (layer "F.Cu") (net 1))
 (segment (start 254.185 62.075) (end 256.08 60.18) (width 0.2) (layer "F.Cu") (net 1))
 (segment (start 251.685 62.075) (end 254.185 62.075) (width 0.2) (layer "F.Cu") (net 1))
 (segment (start 236.685 47.685) (end 236.5 47.5) (width 0.2) (layer "F.Cu") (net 1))
 (segment (start 237.5 47.5) (end 237.5 60.39) (width 0.2) (layer "F.Cu") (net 2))
 (segment (start 237.5 60.39) (end 239.185 62.075) (width 0.2) (layer "F.Cu") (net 2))
 (segment (start 238.5 56.39) (end 238.5 47.5) (width 0.2) (layer "B.Cu") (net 4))
 (segment (start 244.185 62.075) (end 238.5 56.39) (width 0.2) (layer "B.Cu") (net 4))
 (segment (start 253.54 50) (end 253.54 31.33) (width 0.2) (layer "F.Cu") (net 6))
 (segment (start 253.54 31.33) (end 253.21 31) (width 0.2) (layer "F.Cu") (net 6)))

